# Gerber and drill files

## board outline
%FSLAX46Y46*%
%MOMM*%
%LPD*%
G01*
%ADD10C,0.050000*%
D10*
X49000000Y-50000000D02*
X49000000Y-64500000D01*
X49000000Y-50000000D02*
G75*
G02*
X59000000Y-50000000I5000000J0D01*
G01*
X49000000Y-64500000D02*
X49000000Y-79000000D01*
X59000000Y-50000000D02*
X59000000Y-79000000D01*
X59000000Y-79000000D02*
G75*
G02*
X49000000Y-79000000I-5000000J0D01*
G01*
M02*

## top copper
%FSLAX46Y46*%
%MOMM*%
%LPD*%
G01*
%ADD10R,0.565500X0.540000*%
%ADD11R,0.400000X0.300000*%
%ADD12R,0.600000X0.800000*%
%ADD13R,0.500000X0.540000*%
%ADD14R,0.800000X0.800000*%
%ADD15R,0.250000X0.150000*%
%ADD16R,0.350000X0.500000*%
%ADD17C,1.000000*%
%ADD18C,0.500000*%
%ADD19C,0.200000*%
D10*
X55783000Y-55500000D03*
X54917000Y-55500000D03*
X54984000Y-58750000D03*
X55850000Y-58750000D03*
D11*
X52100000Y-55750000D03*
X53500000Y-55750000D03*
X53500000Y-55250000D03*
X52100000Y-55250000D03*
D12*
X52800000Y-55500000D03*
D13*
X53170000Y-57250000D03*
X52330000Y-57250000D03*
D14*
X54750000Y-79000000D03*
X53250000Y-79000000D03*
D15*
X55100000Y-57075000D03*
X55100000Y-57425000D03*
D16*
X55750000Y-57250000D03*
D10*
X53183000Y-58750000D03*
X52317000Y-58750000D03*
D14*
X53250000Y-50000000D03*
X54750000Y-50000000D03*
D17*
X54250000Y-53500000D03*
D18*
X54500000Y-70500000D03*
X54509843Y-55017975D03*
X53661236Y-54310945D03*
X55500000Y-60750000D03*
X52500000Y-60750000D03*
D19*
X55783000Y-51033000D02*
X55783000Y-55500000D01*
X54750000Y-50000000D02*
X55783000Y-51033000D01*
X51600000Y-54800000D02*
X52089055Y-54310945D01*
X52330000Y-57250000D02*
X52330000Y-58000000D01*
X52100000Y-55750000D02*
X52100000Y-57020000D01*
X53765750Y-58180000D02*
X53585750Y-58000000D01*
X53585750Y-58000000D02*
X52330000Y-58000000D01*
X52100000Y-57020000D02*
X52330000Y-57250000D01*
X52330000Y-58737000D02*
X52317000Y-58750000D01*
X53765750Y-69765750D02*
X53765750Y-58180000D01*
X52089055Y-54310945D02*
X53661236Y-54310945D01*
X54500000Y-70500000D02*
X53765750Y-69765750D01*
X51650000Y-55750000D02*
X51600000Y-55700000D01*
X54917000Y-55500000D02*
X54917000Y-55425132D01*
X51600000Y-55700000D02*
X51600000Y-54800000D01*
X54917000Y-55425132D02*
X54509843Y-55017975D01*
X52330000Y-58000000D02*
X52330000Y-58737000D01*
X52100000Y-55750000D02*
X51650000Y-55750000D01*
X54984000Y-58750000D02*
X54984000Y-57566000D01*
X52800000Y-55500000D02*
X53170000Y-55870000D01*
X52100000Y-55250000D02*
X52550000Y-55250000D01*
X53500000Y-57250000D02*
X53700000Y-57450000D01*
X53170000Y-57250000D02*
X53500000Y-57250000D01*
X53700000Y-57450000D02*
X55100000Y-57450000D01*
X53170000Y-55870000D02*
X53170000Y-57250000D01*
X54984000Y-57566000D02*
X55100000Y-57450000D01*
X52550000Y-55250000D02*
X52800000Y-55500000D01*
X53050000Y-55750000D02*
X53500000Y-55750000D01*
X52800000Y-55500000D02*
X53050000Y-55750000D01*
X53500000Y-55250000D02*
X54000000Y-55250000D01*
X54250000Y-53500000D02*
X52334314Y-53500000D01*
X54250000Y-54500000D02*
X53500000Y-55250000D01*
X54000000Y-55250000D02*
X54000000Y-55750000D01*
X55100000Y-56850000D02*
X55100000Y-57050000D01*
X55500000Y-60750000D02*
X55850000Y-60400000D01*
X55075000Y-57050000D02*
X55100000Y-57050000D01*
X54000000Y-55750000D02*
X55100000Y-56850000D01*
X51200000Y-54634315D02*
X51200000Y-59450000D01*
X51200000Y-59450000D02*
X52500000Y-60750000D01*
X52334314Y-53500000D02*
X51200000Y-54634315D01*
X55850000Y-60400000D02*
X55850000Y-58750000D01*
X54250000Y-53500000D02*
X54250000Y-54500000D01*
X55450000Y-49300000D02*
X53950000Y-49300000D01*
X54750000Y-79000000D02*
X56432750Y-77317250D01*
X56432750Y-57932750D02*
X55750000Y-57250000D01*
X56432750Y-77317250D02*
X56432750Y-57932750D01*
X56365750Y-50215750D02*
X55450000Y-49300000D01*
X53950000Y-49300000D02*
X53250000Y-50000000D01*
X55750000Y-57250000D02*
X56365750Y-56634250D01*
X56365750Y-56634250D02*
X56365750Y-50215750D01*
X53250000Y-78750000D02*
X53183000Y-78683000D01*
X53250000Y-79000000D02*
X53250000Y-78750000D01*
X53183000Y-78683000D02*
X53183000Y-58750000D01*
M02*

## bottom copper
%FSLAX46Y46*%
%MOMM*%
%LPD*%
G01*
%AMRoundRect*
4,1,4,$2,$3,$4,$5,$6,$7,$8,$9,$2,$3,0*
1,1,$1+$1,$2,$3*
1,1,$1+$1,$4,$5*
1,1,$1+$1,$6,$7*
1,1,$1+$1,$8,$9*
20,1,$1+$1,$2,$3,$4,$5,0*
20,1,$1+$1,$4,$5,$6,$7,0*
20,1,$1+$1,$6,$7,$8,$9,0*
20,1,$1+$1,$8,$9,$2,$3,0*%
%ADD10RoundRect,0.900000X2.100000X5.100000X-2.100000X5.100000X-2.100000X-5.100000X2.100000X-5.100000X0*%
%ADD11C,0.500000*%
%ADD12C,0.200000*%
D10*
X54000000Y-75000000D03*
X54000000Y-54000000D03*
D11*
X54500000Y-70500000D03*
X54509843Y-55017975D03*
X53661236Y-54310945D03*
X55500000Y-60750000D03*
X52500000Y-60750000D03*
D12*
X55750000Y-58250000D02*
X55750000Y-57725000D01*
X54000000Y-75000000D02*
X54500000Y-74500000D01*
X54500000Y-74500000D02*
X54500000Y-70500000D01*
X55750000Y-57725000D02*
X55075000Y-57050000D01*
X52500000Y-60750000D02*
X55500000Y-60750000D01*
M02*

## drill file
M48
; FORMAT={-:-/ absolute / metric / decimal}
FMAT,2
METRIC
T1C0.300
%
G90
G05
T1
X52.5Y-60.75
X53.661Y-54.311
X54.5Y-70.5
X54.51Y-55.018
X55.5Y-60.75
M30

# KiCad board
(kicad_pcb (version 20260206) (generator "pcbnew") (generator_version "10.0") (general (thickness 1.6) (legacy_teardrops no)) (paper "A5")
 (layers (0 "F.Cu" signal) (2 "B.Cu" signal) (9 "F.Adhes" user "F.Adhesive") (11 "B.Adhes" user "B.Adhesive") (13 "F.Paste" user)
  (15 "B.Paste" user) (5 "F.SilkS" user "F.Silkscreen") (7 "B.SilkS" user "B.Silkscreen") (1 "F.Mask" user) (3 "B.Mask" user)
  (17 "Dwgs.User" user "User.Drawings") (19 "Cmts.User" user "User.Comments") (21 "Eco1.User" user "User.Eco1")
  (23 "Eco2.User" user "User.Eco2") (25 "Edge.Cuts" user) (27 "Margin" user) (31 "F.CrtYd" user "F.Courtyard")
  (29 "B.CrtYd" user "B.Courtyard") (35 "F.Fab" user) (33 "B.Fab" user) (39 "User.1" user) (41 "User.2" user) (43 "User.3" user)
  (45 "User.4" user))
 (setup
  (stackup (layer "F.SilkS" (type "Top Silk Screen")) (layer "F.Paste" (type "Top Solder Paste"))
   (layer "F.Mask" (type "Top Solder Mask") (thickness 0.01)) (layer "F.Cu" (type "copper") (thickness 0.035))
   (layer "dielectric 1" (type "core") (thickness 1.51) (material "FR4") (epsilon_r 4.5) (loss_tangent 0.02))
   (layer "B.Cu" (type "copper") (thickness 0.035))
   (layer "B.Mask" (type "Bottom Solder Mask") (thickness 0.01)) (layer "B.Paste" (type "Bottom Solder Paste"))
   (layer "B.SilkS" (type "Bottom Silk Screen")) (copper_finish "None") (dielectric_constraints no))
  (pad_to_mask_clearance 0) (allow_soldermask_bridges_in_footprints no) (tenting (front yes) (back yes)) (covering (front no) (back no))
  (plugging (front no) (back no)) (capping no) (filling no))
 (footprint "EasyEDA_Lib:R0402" (layer "F.Cu") (at 55.35 55.5 180)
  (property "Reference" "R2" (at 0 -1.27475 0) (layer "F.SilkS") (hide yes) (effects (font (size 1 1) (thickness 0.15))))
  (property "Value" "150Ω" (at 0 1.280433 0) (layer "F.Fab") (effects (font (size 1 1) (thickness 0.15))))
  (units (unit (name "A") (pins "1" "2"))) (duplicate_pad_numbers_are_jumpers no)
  (pad "1" smd rect (at -0.433 0 180) (size 0.5655 0.54) (layers "F.Cu" "F.Mask" "F.Paste") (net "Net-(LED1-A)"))
  (pad "2" smd rect (at 0.433 0 180) (size 0.5655 0.54) (layers "F.Cu" "F.Mask" "F.Paste") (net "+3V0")))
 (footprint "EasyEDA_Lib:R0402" (layer "F.Cu") (at 55.417 58.75)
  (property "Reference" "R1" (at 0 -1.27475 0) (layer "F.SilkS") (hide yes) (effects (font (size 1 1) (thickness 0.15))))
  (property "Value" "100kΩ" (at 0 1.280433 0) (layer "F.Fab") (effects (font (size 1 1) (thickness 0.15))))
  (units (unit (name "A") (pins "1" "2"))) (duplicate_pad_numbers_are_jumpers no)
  (pad "1" smd rect (at -0.433 0) (size 0.5655 0.54) (layers "F.Cu" "F.Mask" "F.Paste") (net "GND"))
  (pad "2" smd rect (at 0.433 0) (size 0.5655 0.54) (layers "F.Cu" "F.Mask" "F.Paste") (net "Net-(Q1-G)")))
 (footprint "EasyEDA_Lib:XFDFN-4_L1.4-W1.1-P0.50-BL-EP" (layer "F.Cu") (at 52.8 55.5)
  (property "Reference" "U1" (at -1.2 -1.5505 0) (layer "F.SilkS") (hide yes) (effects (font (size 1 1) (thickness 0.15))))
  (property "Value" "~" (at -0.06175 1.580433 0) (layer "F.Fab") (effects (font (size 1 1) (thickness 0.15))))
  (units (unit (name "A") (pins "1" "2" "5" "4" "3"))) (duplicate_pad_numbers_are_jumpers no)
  (pad "1" smd rect (at -0.7 0.25 270) (size 0.3 0.4) (layers "F.Cu" "F.Mask" "F.Paste") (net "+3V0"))
  (pad "2" smd rect (at 0.7 0.25 90) (size 0.3 0.4) (layers "F.Cu" "F.Mask" "F.Paste") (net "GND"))
  (pad "3" smd rect (at 0.7 -0.25 90) (size 0.3 0.4) (layers "F.Cu" "F.Mask" "F.Paste") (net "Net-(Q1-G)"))
  (pad "4" smd rect (at -0.7 -0.25 90) (size 0.3 0.4) (layers "F.Cu" "F.Mask" "F.Paste") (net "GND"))
  (pad "5" smd rect (at 0 0 270) (size 0.8 0.6) (layers "F.Cu" "F.Mask" "F.Paste") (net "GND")))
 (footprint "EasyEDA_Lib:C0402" (layer "F.Cu") (at 52.75 57.25 180)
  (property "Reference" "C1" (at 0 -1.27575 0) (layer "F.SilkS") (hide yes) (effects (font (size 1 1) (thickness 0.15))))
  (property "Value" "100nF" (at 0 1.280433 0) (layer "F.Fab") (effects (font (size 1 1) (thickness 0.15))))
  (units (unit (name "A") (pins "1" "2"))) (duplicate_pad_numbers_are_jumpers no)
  (pad "1" smd rect (at -0.42 0 180) (size 0.5 0.54) (layers "F.Cu" "F.Mask" "F.Paste") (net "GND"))
  (pad "2" smd rect (at 0.42 0 180) (size 0.5 0.54) (layers "F.Cu" "F.Mask" "F.Paste") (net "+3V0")))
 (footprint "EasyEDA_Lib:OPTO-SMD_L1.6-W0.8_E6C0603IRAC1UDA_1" (layer "F.Cu") (at 54 79 180)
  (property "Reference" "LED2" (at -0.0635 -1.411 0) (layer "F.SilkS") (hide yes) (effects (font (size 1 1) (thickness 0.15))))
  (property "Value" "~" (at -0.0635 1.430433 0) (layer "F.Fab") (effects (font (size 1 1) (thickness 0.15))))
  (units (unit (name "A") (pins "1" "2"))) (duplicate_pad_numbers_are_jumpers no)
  (pad "1" smd rect (at -0.75 0 180) (size 0.8 0.8) (layers "F.Cu" "F.Mask" "F.Paste") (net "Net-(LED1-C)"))
  (pad "2" smd rect (at 0.75 0 180) (size 0.8 0.8) (layers "F.Cu" "F.Mask" "F.Paste") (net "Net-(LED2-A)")))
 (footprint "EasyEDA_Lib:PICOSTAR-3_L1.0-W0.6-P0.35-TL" (layer "F.Cu") (at 55.425 57.25)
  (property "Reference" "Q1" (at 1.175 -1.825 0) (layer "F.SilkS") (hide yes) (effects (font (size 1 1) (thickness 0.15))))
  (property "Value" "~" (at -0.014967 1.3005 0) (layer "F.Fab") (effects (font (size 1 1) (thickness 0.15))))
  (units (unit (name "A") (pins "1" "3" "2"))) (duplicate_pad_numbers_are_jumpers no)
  (pad "1" smd rect (at -0.325 -0.175 270) (size 0.15 0.25) (layers "F.Cu" "F.Mask" "F.Paste") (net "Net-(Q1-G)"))
  (pad "2" smd rect (at -0.325 0.175 270) (size 0.15 0.25) (layers "F.Cu" "F.Mask" "F.Paste") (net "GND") (clearance 0.2))
  (pad "3" smd rect (at 0.325 0 180) (size 0.35 0.5) (layers "F.Cu" "F.Mask" "F.Paste") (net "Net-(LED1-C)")))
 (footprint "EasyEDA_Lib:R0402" (layer "F.Cu") (at 52.75 58.75 180)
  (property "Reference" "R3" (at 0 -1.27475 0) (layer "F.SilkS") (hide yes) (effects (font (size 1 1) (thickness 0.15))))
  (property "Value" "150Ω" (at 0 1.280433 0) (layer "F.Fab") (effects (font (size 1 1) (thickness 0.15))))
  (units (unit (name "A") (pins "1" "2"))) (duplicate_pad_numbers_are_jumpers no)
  (pad "1" smd rect (at -0.433 0 180) (size 0.5655 0.54) (layers "F.Cu" "F.Mask" "F.Paste") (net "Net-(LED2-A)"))
  (pad "2" smd rect (at 0.433 0 180) (size 0.5655 0.54) (layers "F.Cu" "F.Mask" "F.Paste") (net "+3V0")))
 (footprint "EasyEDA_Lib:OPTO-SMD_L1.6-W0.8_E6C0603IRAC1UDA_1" (layer "F.Cu") (at 54 50)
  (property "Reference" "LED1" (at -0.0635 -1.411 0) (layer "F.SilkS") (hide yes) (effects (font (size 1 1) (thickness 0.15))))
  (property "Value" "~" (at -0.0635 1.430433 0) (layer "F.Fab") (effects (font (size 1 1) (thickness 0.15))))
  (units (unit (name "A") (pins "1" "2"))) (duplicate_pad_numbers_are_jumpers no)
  (pad "1" smd rect (at -0.75 0) (size 0.8 0.8) (layers "F.Cu" "F.Mask" "F.Paste") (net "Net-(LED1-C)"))
  (pad "2" smd rect (at 0.75 0) (size 0.8 0.8) (layers "F.Cu" "F.Mask" "F.Paste") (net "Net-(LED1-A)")))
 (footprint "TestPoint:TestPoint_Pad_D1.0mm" (layer "F.Cu") (at 54.25 53.5)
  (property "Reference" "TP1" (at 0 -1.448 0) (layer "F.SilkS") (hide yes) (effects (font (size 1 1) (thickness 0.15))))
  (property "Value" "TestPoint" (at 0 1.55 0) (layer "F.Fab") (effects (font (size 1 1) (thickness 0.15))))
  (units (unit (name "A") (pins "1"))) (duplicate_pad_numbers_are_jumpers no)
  (pad "1" smd circle (at 0 0) (size 1 1) (layers "F.Cu" "F.Mask") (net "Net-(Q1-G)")))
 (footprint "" (layer "F.Cu") (at 54 75)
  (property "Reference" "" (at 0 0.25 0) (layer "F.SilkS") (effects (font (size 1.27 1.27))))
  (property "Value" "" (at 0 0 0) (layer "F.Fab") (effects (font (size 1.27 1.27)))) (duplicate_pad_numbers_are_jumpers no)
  (pad "1" connect roundrect (at 0 0 180) (size 6 12) (layers "B.Cu" "B.Mask") (roundrect_rratio 0.15) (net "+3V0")))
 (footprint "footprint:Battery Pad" (layer "B.Cu") (at 54 54 180)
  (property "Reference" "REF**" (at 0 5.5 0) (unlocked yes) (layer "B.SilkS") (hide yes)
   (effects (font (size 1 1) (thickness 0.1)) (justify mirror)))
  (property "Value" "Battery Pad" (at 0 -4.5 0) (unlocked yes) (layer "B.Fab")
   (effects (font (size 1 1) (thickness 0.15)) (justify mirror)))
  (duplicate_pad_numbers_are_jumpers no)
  (pad "1" connect roundrect (at 0 0 180) (size 6 12) (layers "B.Cu" "B.Mask") (roundrect_rratio 0.15) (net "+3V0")))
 (gr_line (start 49 50) (end 49 64.5) (stroke (width 0.05) (type default)) (layer "Edge.Cuts"))
 (gr_arc (start 49 50) (mid 54 45) (end 59 50) (stroke (width 0.05) (type default)) (layer "Edge.Cuts"))
 (gr_line (start 49 64.5) (end 49 79) (stroke (width 0.05) (type default)) (layer "Edge.Cuts"))
 (gr_line (start 59 50) (end 59 79) (stroke (width 0.05) (type default)) (layer "Edge.Cuts"))
 (gr_arc (start 59 79) (mid 54 84) (end 49 79) (stroke (width 0.05) (type default)) (layer "Edge.Cuts"))
 (segment (start 55.783 51.033) (end 55.783 55.5) (width 0.2) (layer "F.Cu") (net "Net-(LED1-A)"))
 (segment (start 54.75 50) (end 55.783 51.033) (width 0.2) (layer "F.Cu") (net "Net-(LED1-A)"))
 (segment (start 51.6 54.8) (end 52.089055 54.310945) (width 0.2) (layer "F.Cu") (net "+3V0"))
 (segment (start 52.33 57.25) (end 52.33 58) (width 0.2) (layer "F.Cu") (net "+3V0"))
 (segment (start 52.1 55.75) (end 52.1 57.02) (width 0.2) (layer "F.Cu") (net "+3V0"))
 (segment (start 53.76575 58.18) (end 53.58575 58) (width 0.2) (layer "F.Cu") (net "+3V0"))
 (segment (start 53.58575 58) (end 52.33 58) (width 0.2) (layer "F.Cu") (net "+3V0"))
 (segment (start 52.1 57.02) (end 52.33 57.25) (width 0.2) (layer "F.Cu") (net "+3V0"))
 (segment (start 52.33 58.737) (end 52.317 58.75) (width 0.2) (layer "F.Cu") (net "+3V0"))
 (segment (start 53.76575 69.76575) (end 53.76575 58.18) (width 0.2) (layer "F.Cu") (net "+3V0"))
 (segment (start 52.089055 54.310945) (end 53.661236 54.310945) (width 0.2) (layer "F.Cu") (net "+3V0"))
 (segment (start 54.5 70.5) (end 53.76575 69.76575) (width 0.2) (layer "F.Cu") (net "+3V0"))
 (segment (start 51.65 55.75) (end 51.6 55.7) (width 0.2) (layer "F.Cu") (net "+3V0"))
 (segment (start 54.917 55.5) (end 54.917 55.425132) (width 0.2) (layer "F.Cu") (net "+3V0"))
 (segment (start 51.6 55.7) (end 51.6 54.8) (width 0.2) (layer "F.Cu") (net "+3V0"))
 (segment (start 54.917 55.425132) (end 54.509843 55.017975) (width 0.2) (layer "F.Cu") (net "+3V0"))
 (segment (start 52.33 58) (end 52.33 58.737) (width 0.2) (layer "F.Cu") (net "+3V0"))
 (segment (start 52.1 55.75) (end 51.65 55.75) (width 0.2) (layer "F.Cu") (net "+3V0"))
 (via (at 54.5 70.5) (size 0.5) (drill 0.3) (layers "F.Cu" "B.Cu") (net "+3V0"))
 (via (at 54.509843 55.017975) (size 0.5) (drill 0.3) (layers "F.Cu" "B.Cu") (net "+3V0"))
 (via (at 53.661236 54.310945) (size 0.5) (drill 0.3) (layers "F.Cu" "B.Cu") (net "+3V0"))
 (segment (start 55.75 58.25) (end 55.75 57.725) (width 0.2) (layer "B.Cu") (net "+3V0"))
 (segment (start 54 75) (end 54.5 74.5) (width 0.2) (layer "B.Cu") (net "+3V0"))
 (segment (start 54.5 74.5) (end 54.5 70.5) (width 0.2) (layer "B.Cu") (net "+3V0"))
 (segment (start 55.75 57.725) (end 55.075 57.05) (width 0.2) (layer "B.Cu") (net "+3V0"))
 (segment (start 54.984 58.75) (end 54.984 57.566) (width 0.2) (layer "F.Cu") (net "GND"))
 (segment (start 52.8 55.5) (end 53.17 55.87) (width 0.2) (layer "F.Cu") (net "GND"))
 (segment (start 52.1 55.25) (end 52.55 55.25) (width 0.2) (layer "F.Cu") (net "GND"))
 (segment (start 53.5 57.25) (end 53.7 57.45) (width 0.2) (layer "F.Cu") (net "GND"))
 (segment (start 53.17 57.25) (end 53.5 57.25) (width 0.2) (layer "F.Cu") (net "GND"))
 (segment (start 53.7 57.45) (end 55.1 57.45) (width 0.2) (layer "F.Cu") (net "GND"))
 (segment (start 53.17 55.87) (end 53.17 57.25) (width 0.2) (layer "F.Cu") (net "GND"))
 (segment (start 54.984 57.566) (end 55.1 57.45) (width 0.2) (layer "F.Cu") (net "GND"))
 (segment (start 52.55 55.25) (end 52.8 55.5) (width 0.2) (layer "F.Cu") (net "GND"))
 (segment (start 53.05 55.75) (end 53.5 55.75) (width 0.2) (layer "F.Cu") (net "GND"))
 (segment (start 52.8 55.5) (end 53.05 55.75) (width 0.2) (layer "F.Cu") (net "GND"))
 (segment (start 53.5 55.25) (end 54 55.25) (width 0.2) (layer "F.Cu") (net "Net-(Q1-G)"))
 (segment (start 54.25 53.5) (end 52.334314 53.5) (width 0.2) (layer "F.Cu") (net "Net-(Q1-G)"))
 (segment (start 54.25 54.5) (end 53.5 55.25) (width 0.2) (layer "F.Cu") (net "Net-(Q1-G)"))
 (segment (start 54 55.25) (end 54 55.75) (width 0.2) (layer "F.Cu") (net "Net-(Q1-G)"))
 (segment (start 55.1 56.85) (end 55.1 57.05) (width 0.2) (layer "F.Cu") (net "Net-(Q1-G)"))
 (segment (start 55.5 60.75) (end 55.85 60.4) (width 0.2) (layer "F.Cu") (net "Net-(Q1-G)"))
 (segment (start 55.075 57.05) (end 55.1 57.05) (width 0.2) (layer "F.Cu") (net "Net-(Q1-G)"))
 (segment (start 54 55.75) (end 55.1 56.85) (width 0.2) (layer "F.Cu") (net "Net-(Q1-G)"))
 (segment (start 51.2 54.634315) (end 51.2 59.45) (width 0.2) (layer "F.Cu") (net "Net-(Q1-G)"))
 (segment (start 51.2 59.45) (end 52.5 60.75) (width 0.2) (layer "F.Cu") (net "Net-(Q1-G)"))
 (segment (start 52.334314 53.5) (end 51.2 54.634315) (width 0.2) (layer "F.Cu") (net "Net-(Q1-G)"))
 (segment (start 55.85 60.4) (end 55.85 58.75) (width 0.2) (layer "F.Cu") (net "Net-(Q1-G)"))
 (segment (start 54.25 53.5) (end 54.25 54.5) (width 0.2) (layer "F.Cu") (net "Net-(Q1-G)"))
 (via (at 55.5 60.75) (size 0.5) (drill 0.3) (layers "F.Cu" "B.Cu") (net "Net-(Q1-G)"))
 (via (at 52.5 60.75) (size 0.5) (drill 0.3) (layers "F.Cu" "B.Cu") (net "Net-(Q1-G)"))
 (segment (start 52.5 60.75) (end 55.5 60.75) (width 0.2) (layer "B.Cu") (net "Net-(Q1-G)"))
 (segment (start 55.45 49.3) (end 53.95 49.3) (width 0.2) (layer "F.Cu") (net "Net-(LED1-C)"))
 (segment (start 54.75 79) (end 56.43275 77.31725) (width 0.2) (layer "F.Cu") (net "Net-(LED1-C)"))
 (segment (start 56.43275 57.93275) (end 55.75 57.25) (width 0.2) (layer "F.Cu") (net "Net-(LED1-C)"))
 (segment (start 56.43275 77.31725) (end 56.43275 57.93275) (width 0.2) (layer "F.Cu") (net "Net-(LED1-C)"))
 (segment (start 56.36575 50.21575) (end 55.45 49.3) (width 0.2) (layer "F.Cu") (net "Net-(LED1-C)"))
 (segment (start 53.95 49.3) (end 53.25 50) (width 0.2) (layer "F.Cu") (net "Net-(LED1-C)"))
 (segment (start 55.75 57.25) (end 56.36575 56.63425) (width 0.2) (layer "F.Cu") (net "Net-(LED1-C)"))
 (segment (start 56.36575 56.63425) (end 56.36575 50.21575) (width 0.2) (layer "F.Cu") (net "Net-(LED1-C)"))
 (segment (start 53.25 78.75) (end 53.183 78.683) (width 0.2) (layer "F.Cu") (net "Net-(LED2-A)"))
 (segment (start 53.25 79) (end 53.25 78.75) (width 0.2) (layer "F.Cu") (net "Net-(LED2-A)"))
 (segment (start 53.183 78.683) (end 53.183 58.75) (width 0.2) (layer "F.Cu") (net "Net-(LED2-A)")))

